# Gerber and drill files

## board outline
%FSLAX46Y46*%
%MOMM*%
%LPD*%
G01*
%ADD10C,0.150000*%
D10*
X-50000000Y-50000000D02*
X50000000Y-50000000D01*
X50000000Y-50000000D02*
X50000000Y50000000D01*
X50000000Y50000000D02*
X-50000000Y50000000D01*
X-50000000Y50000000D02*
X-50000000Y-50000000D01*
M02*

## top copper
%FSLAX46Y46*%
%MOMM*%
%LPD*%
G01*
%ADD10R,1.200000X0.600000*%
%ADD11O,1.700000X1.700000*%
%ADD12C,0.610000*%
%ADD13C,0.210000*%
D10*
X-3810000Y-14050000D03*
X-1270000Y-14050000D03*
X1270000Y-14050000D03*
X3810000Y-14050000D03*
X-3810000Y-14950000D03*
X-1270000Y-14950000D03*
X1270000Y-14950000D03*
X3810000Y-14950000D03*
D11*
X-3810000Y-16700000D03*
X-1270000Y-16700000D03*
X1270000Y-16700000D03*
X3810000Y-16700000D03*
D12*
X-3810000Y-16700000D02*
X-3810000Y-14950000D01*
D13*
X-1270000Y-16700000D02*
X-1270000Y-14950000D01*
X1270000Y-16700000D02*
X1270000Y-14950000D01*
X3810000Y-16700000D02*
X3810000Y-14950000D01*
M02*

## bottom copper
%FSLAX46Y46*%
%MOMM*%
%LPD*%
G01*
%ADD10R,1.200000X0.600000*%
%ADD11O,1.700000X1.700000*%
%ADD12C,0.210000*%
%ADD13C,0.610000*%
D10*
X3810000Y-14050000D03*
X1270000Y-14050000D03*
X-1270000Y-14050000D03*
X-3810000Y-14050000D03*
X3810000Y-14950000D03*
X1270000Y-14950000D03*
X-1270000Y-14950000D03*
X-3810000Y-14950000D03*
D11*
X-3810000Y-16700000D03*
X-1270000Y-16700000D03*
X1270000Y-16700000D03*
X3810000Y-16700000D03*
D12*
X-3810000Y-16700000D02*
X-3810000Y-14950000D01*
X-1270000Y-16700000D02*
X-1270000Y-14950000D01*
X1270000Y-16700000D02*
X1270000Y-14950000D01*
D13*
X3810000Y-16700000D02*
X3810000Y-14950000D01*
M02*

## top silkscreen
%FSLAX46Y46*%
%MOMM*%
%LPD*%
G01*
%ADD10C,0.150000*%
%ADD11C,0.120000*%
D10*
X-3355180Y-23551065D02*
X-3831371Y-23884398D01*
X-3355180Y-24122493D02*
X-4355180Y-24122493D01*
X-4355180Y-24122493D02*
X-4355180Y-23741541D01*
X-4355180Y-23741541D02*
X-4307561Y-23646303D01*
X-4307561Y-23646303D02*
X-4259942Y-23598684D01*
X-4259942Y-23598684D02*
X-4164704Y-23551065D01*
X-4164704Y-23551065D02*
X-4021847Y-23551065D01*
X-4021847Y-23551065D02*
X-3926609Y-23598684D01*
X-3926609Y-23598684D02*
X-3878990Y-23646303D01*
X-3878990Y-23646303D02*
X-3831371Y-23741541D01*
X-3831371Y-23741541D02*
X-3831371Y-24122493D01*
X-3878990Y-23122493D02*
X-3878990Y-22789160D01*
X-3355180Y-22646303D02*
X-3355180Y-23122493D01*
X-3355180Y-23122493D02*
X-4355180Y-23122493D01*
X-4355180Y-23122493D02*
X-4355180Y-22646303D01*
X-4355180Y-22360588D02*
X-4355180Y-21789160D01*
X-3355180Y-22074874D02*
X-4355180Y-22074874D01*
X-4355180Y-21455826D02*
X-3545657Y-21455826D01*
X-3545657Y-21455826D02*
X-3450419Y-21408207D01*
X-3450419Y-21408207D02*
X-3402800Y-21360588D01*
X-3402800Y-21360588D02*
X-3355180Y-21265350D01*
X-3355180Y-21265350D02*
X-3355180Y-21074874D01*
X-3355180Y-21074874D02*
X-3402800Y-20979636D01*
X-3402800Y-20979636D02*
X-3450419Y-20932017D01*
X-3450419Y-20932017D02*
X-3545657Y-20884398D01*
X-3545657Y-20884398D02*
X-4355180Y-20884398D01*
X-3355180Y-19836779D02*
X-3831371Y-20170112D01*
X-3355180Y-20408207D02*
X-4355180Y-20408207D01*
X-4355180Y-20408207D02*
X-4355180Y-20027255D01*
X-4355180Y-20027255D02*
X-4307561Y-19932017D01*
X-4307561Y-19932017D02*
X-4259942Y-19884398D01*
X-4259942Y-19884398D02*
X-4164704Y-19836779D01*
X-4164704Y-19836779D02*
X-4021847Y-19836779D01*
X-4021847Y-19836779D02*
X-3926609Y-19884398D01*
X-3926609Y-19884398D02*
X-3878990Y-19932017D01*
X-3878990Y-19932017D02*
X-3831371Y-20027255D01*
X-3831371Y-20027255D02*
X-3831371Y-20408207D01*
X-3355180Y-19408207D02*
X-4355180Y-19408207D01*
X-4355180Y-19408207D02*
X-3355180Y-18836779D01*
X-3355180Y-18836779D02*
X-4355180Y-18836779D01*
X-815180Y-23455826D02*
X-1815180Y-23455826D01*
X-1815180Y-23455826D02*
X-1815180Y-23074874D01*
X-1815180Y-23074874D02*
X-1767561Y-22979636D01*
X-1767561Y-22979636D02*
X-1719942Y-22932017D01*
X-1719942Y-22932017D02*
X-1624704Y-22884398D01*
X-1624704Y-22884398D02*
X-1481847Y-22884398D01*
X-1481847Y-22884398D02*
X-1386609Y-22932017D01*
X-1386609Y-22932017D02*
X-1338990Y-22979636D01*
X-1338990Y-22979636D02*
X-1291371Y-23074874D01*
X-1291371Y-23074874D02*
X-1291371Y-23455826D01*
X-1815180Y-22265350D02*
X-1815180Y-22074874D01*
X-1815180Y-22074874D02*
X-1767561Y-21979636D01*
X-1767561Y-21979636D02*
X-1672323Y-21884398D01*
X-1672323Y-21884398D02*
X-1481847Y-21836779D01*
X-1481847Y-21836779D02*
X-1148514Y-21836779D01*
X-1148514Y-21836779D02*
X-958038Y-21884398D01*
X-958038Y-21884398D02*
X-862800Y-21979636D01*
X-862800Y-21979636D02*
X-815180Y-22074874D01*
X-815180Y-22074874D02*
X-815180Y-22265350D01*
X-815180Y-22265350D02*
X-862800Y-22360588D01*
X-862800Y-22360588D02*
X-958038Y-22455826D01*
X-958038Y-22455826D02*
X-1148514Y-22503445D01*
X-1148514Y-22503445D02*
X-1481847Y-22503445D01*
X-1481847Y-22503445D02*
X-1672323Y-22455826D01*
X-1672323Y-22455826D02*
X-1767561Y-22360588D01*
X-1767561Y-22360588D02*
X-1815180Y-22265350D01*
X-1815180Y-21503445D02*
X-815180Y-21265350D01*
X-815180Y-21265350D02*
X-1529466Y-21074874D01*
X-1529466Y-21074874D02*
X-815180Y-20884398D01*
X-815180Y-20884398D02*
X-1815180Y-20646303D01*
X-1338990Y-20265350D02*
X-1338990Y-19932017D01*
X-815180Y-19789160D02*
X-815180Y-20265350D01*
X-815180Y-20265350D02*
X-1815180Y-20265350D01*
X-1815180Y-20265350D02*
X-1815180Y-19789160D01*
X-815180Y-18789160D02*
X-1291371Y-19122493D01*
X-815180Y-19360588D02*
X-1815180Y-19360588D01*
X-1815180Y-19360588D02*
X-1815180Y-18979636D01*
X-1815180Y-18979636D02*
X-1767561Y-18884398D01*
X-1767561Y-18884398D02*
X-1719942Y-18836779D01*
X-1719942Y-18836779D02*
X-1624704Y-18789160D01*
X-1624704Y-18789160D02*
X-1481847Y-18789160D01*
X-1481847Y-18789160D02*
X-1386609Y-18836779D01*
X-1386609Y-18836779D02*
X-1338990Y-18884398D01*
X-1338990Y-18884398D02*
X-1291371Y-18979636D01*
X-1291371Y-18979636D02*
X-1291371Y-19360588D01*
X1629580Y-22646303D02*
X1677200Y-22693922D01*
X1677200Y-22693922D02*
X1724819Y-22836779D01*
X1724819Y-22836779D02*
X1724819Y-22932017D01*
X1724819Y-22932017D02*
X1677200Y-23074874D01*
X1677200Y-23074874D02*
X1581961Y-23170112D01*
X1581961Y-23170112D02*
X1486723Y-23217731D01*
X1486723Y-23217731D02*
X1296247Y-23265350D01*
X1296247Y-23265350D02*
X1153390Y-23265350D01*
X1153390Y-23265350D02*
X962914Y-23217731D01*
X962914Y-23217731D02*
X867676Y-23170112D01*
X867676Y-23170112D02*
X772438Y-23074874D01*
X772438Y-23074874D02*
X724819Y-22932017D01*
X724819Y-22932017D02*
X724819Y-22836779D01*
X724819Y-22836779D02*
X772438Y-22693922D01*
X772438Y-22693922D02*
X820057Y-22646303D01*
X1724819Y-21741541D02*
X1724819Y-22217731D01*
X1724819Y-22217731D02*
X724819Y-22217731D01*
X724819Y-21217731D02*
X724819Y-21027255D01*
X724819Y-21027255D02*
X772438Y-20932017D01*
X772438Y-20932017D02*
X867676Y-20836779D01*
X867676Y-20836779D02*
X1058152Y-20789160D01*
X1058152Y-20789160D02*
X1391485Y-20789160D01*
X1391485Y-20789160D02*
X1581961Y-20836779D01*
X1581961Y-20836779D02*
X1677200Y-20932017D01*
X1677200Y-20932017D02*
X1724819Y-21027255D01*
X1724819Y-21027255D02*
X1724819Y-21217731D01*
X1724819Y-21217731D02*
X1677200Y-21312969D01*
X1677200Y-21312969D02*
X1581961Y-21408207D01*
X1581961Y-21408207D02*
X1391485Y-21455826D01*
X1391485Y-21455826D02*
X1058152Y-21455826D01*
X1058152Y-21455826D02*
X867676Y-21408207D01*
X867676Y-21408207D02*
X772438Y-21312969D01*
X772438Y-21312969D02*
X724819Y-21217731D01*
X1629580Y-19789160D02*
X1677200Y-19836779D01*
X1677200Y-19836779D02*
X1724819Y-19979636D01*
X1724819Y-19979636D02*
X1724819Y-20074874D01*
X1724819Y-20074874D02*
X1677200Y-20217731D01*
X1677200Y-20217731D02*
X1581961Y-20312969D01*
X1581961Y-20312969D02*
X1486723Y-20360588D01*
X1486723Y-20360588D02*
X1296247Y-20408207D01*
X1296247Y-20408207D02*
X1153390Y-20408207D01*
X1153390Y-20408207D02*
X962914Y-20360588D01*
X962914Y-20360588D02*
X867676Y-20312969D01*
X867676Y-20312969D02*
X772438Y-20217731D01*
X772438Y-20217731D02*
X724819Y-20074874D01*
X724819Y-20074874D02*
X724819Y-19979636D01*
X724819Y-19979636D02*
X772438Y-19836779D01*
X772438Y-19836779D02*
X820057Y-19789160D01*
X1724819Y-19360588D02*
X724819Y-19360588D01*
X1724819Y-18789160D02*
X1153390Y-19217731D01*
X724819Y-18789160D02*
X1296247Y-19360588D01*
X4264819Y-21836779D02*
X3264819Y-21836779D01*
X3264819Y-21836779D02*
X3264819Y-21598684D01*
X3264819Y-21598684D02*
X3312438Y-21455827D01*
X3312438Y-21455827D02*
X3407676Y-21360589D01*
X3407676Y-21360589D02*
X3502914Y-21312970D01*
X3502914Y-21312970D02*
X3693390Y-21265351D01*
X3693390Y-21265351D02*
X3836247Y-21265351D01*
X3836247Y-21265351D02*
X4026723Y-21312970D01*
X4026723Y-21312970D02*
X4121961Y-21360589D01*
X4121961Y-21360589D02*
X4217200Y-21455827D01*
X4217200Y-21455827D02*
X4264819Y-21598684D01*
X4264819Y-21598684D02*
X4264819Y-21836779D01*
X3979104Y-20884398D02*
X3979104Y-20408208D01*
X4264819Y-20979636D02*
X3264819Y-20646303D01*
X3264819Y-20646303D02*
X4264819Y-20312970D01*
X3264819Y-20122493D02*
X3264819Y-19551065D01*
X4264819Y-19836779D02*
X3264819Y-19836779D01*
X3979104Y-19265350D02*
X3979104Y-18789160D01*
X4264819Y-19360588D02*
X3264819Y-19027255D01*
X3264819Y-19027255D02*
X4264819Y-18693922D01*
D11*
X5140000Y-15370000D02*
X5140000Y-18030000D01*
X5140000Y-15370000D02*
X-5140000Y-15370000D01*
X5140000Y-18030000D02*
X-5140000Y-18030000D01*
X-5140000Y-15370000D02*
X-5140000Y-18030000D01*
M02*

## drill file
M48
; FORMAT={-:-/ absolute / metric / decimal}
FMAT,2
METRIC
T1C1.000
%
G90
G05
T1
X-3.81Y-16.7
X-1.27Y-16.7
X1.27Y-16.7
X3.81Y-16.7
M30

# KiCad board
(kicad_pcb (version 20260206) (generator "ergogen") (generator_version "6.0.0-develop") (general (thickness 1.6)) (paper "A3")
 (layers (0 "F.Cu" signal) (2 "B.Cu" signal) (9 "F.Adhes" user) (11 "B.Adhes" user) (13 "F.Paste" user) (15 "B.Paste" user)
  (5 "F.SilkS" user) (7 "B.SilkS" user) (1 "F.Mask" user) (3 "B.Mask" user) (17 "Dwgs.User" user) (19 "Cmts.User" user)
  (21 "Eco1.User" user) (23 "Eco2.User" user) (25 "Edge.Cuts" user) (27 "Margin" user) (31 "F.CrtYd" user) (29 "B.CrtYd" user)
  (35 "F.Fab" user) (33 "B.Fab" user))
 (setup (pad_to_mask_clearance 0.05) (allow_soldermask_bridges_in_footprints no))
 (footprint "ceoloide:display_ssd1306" (layer "F.Cu") (at 0 0 0)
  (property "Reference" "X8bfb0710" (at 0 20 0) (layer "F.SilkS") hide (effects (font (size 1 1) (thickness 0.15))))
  (fp_line (start 5.14 15.37) (end 5.14 18.03) (layer "F.SilkS") (stroke (width 0.12) (type solid)))
  (fp_line (start 5.14 15.37) (end -5.14 15.37) (layer "F.SilkS") (stroke (width 0.12) (type solid)))
  (fp_line (start 5.14 18.03) (end -5.14 18.03) (layer "F.SilkS") (stroke (width 0.12) (type solid)))
  (fp_line (start -5.14 15.37) (end -5.14 18.03) (layer "F.SilkS") (stroke (width 0.12) (type solid)))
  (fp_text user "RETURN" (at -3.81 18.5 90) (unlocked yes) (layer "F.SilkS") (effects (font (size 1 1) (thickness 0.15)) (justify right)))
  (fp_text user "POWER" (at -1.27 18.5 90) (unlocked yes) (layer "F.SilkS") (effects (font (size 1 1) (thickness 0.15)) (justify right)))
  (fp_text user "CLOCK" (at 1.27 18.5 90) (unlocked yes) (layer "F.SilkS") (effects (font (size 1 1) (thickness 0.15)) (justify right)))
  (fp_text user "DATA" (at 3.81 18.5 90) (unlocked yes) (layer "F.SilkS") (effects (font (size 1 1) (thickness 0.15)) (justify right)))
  (pad "14" smd rect (at -3.81 14.05 90) (size 0.6 1.2) (layers "F.Cu" "F.Paste" "F.Mask") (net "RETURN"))
  (pad "15" smd rect (at -1.27 14.05 90) (size 0.6 1.2) (layers "F.Cu" "F.Paste" "F.Mask") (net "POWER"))
  (pad "16" smd rect (at 1.27 14.05 90) (size 0.6 1.2) (layers "F.Cu" "F.Paste" "F.Mask") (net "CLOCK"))
  (pad "17" smd rect (at 3.81 14.05 90) (size 0.6 1.2) (layers "F.Cu" "F.Paste" "F.Mask") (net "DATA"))
  (pad "10" smd rect (at -3.81 14.95 90) (size 0.6 1.2) (layers "F.Cu" "F.Paste" "F.Mask") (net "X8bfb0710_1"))
  (pad "11" smd rect (at -1.27 14.95 90) (size 0.6 1.2) (layers "F.Cu" "F.Paste" "F.Mask") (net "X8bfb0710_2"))
  (pad "12" smd rect (at 1.27 14.95 90) (size 0.6 1.2) (layers "F.Cu" "F.Paste" "F.Mask") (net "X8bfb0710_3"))
  (pad "13" smd rect (at 3.81 14.95 90) (size 0.6 1.2) (layers "F.Cu" "F.Paste" "F.Mask") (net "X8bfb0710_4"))
  (pad "24" smd rect (at 3.81 14.05 270) (size 0.6 1.2) (layers "B.Cu" "B.Paste" "B.Mask") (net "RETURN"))
  (pad "25" smd rect (at 1.27 14.05 270) (size 0.6 1.2) (layers "B.Cu" "B.Paste" "B.Mask") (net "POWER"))
  (pad "26" smd rect (at -1.27 14.05 270) (size 0.6 1.2) (layers "B.Cu" "B.Paste" "B.Mask") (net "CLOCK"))
  (pad "27" smd rect (at -3.81 14.05 270) (size 0.6 1.2) (layers "B.Cu" "B.Paste" "B.Mask") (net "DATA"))
  (pad "20" smd rect (at 3.81 14.95 270) (size 0.6 1.2) (layers "B.Cu" "B.Paste" "B.Mask") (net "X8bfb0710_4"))
  (pad "21" smd rect (at 1.27 14.95 270) (size 0.6 1.2) (layers "B.Cu" "B.Paste" "B.Mask") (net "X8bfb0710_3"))
  (pad "22" smd rect (at -1.27 14.95 270) (size 0.6 1.2) (layers "B.Cu" "B.Paste" "B.Mask") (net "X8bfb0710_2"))
  (pad "23" smd rect (at -3.81 14.95 270) (size 0.6 1.2) (layers "B.Cu" "B.Paste" "B.Mask") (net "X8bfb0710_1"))
  (pad "1" thru_hole oval (at -3.81 16.7 270) (size 1.7 1.7) (drill 1) (layers "*.Cu" "*.Mask") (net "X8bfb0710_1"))
  (pad "2" thru_hole oval (at -1.27 16.7 270) (size 1.7 1.7) (drill 1) (layers "*.Cu" "*.Mask") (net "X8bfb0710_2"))
  (pad "3" thru_hole oval (at 1.27 16.7 270) (size 1.7 1.7) (drill 1) (layers "*.Cu" "*.Mask") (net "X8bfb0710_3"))
  (pad "4" thru_hole oval (at 3.81 16.7 270) (size 1.7 1.7) (drill 1) (layers "*.Cu" "*.Mask") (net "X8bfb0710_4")))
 (segment (start -3.81 16.7) (end -3.81 14.95) (width 0.61) (layer "F.Cu") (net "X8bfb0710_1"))
 (segment (start -1.27 16.7) (end -1.27 14.95) (width 0.21) (layer "F.Cu") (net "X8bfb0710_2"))
 (segment (start 1.27 16.7) (end 1.27 14.95) (width 0.21) (layer "F.Cu") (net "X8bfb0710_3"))
 (segment (start 3.81 16.7) (end 3.81 14.95) (width 0.21) (layer "F.Cu") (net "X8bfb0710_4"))
 (segment (start -3.81 16.7) (end -3.81 14.95) (width 0.21) (layer "B.Cu") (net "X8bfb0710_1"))
 (segment (start -1.27 16.7) (end -1.27 14.95) (width 0.21) (layer "B.Cu") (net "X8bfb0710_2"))
 (segment (start 1.27 16.7) (end 1.27 14.95) (width 0.21) (layer "B.Cu") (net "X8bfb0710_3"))
 (segment (start 3.81 16.7) (end 3.81 14.95) (width 0.61) (layer "B.Cu") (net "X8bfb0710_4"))
 (gr_line (start -50 50) (end 50 50) (layer Edge.Cuts) (stroke (width 0.15) (type default)))
 (gr_line (start 50 50) (end 50 -50) (layer Edge.Cuts) (stroke (width 0.15) (type default)))
 (gr_line (start 50 -50) (end -50 -50) (layer Edge.Cuts) (stroke (width 0.15) (type default)))
 (gr_line (start -50 -50) (end -50 50) (layer Edge.Cuts) (stroke (width 0.15) (type default))))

